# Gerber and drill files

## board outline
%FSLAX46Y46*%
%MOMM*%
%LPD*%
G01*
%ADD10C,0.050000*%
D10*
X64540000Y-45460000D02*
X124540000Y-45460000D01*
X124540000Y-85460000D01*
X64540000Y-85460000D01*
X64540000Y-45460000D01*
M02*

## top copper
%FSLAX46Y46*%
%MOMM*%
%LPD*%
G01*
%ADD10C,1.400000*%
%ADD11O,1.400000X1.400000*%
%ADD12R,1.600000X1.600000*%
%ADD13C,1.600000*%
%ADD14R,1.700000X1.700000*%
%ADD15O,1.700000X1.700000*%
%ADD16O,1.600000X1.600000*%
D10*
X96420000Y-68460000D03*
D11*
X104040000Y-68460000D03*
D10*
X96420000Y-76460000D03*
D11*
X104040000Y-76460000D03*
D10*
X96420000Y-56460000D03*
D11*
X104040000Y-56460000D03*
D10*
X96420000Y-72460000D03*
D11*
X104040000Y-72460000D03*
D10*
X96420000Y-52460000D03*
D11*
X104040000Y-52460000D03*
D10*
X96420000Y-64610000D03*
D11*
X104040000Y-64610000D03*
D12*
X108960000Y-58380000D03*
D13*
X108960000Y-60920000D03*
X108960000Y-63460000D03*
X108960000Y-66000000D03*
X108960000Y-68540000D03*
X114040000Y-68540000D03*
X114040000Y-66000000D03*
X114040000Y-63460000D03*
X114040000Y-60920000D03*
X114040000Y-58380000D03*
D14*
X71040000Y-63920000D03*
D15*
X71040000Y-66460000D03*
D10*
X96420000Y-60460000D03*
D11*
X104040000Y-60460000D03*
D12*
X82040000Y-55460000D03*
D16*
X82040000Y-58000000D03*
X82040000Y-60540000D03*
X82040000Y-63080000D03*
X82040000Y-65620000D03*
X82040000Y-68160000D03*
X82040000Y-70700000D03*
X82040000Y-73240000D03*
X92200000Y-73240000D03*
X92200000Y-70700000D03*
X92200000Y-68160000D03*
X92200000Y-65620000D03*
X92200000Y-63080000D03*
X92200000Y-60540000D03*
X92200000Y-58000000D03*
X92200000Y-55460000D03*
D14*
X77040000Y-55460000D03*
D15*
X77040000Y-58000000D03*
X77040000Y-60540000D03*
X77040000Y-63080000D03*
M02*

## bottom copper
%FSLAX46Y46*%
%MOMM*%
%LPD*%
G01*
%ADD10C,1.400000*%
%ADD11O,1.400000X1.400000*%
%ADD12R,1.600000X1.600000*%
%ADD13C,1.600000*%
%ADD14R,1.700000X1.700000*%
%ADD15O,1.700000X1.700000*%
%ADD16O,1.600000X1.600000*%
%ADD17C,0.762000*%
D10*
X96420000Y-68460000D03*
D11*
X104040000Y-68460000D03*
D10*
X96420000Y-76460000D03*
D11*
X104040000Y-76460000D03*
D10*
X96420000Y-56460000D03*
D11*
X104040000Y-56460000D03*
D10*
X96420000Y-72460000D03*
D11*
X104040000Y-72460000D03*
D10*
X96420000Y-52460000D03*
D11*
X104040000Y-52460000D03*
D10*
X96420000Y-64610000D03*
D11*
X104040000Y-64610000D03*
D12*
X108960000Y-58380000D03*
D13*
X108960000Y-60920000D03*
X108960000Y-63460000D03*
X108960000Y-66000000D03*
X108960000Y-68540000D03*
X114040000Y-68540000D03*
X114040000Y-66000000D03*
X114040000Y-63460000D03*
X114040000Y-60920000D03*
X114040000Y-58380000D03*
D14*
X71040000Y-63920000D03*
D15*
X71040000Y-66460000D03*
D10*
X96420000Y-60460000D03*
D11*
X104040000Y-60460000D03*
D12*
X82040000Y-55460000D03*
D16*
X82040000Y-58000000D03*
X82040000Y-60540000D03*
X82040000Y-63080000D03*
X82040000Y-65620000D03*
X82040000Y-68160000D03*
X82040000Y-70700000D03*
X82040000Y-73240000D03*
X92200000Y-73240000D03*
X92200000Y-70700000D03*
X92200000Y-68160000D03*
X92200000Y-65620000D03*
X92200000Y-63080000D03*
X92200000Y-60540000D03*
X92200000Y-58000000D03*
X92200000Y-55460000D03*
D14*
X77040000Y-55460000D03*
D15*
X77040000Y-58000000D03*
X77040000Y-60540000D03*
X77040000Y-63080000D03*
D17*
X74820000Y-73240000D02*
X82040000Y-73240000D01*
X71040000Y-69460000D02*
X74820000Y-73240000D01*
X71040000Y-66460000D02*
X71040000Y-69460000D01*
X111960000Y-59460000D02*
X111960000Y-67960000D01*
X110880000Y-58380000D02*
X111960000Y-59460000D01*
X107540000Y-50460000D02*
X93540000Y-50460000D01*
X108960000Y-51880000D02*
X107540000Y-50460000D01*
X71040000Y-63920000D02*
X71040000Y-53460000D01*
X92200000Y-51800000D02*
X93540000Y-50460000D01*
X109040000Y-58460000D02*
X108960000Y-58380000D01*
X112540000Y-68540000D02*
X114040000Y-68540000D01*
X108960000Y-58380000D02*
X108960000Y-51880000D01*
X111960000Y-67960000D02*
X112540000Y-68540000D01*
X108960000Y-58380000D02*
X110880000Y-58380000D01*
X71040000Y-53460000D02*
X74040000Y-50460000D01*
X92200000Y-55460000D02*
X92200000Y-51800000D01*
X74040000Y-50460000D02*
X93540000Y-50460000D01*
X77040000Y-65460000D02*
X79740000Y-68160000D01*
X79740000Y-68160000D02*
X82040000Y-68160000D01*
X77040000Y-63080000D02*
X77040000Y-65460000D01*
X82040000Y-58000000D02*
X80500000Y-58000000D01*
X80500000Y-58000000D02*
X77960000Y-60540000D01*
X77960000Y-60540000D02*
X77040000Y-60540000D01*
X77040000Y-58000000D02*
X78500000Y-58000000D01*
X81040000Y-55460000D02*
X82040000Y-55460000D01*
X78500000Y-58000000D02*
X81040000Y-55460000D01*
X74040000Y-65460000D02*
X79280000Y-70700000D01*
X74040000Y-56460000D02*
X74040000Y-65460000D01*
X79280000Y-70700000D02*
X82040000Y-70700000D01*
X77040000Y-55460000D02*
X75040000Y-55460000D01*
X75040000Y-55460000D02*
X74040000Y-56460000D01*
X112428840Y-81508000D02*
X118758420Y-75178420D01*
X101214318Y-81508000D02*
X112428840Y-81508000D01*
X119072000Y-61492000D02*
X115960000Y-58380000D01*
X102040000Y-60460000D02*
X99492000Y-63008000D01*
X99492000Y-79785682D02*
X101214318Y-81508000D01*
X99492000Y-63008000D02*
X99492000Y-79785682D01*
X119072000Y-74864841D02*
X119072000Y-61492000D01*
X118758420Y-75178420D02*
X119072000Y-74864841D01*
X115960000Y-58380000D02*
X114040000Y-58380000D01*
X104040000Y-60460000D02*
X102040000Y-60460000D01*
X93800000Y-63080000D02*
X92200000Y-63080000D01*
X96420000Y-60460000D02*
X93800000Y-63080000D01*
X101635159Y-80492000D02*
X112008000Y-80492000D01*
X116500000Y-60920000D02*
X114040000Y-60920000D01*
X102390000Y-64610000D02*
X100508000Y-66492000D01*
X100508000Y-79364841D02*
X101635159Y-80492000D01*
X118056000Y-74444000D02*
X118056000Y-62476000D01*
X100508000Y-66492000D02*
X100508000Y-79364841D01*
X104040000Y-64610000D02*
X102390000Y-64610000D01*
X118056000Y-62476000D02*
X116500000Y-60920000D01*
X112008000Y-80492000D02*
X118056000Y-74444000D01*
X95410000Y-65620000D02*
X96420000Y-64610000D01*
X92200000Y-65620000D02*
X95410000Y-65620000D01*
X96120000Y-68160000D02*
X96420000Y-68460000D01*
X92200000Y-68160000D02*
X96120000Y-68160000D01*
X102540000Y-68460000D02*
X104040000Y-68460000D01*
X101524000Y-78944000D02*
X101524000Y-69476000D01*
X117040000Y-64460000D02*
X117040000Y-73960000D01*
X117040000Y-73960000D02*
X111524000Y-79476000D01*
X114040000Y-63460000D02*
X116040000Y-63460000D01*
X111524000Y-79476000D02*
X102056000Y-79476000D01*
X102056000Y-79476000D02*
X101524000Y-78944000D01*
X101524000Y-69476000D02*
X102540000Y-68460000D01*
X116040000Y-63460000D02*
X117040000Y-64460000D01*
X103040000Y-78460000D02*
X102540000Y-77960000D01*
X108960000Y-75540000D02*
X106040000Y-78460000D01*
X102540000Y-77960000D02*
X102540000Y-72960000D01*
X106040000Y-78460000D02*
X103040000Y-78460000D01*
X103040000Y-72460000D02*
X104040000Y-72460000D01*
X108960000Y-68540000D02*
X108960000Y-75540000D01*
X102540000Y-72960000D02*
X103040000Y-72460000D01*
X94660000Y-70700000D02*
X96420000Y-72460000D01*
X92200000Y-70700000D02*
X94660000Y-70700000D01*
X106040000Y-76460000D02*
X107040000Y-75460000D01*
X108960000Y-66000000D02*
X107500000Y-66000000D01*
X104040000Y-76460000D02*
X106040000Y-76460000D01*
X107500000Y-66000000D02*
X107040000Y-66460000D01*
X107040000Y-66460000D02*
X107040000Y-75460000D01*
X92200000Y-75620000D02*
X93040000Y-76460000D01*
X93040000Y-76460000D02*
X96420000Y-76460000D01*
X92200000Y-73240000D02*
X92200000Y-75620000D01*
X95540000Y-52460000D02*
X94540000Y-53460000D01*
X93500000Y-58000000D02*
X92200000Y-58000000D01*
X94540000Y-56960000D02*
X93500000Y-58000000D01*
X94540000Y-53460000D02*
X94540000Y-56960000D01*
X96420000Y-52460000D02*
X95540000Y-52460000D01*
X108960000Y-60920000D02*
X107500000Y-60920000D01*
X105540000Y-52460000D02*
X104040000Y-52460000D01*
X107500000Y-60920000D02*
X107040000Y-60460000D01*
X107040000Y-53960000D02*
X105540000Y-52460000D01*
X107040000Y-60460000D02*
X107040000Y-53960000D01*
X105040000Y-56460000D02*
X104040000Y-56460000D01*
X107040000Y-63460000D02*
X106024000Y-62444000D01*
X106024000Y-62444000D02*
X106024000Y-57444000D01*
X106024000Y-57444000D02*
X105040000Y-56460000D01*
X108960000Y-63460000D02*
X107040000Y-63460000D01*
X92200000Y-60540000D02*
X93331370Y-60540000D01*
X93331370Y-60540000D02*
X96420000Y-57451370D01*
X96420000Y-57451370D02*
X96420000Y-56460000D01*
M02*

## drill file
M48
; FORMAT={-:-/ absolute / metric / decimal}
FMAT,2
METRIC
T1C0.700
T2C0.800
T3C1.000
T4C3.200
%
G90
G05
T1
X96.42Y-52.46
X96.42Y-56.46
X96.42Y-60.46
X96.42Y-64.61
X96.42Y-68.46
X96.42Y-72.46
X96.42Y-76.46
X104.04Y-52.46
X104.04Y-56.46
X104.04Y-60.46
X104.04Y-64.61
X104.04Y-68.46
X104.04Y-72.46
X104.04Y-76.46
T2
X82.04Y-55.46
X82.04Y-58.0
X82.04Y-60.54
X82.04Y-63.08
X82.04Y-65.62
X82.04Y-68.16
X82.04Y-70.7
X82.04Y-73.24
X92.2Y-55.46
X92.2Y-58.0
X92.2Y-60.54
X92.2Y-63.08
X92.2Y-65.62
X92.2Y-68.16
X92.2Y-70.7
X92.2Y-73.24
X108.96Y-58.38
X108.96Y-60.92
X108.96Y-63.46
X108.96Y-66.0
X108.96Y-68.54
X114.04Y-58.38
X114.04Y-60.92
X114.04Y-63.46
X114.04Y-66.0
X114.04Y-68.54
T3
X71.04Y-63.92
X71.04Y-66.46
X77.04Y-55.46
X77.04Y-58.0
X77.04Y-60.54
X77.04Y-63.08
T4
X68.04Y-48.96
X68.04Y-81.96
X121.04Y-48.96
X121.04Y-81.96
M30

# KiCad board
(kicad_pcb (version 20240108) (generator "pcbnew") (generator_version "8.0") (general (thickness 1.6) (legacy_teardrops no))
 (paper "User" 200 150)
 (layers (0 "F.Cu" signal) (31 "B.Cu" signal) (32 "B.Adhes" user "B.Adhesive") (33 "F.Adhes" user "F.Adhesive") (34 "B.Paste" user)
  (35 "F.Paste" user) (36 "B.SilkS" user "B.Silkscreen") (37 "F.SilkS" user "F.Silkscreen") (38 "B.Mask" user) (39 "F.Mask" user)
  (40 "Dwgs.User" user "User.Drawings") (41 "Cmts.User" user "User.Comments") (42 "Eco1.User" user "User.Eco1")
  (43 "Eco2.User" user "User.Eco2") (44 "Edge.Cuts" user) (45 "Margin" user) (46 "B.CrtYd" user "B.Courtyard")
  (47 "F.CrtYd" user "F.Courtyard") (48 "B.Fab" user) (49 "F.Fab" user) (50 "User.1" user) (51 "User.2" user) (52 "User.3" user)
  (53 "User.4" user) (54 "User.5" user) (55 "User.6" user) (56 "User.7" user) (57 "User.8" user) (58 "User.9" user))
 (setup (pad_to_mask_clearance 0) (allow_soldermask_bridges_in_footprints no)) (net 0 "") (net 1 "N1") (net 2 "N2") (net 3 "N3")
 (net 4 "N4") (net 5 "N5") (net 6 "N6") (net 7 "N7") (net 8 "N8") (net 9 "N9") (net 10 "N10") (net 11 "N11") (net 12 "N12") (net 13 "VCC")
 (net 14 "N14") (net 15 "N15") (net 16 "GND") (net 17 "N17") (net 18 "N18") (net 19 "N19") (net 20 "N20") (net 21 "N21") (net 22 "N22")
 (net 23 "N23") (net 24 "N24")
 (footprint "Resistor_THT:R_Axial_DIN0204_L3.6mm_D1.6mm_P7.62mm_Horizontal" (layer "F.Cu") (at 96.42 68.46)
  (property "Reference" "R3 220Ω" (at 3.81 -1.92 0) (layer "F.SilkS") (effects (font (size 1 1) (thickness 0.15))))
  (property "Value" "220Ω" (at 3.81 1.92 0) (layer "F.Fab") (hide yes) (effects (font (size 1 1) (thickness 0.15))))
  (pad "1" thru_hole circle (at 0 0) (size 1.4 1.4) (drill 0.7) (layers "*.Cu" "*.Mask") (remove_unused_layers no) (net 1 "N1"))
  (pad "2" thru_hole oval (at 7.62 0) (size 1.4 1.4) (drill 0.7) (layers "*.Cu" "*.Mask") (remove_unused_layers no) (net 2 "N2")))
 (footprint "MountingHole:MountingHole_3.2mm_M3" (layer "F.Cu") (at 68.04 81.96)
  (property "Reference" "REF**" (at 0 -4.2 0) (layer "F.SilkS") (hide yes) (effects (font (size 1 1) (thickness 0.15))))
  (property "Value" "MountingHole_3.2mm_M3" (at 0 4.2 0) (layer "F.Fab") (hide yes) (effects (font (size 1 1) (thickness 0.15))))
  (pad "" np_thru_hole circle (at 0 0) (size 3.2 3.2) (drill 3.2) (layers "*.Cu" "*.Mask")))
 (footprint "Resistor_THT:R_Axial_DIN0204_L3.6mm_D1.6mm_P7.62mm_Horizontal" (layer "F.Cu") (at 96.42 76.46)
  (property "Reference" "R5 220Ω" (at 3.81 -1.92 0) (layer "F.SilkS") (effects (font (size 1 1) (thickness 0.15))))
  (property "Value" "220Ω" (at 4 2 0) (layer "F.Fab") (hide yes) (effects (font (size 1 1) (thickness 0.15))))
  (pad "1" thru_hole circle (at 0 0) (size 1.4 1.4) (drill 0.7) (layers "*.Cu" "*.Mask") (remove_unused_layers no) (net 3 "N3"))
  (pad "2" thru_hole oval (at 7.62 0) (size 1.4 1.4) (drill 0.7) (layers "*.Cu" "*.Mask") (remove_unused_layers no) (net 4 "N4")))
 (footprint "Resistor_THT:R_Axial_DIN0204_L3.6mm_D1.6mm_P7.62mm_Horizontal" (layer "F.Cu") (at 96.42 56.46)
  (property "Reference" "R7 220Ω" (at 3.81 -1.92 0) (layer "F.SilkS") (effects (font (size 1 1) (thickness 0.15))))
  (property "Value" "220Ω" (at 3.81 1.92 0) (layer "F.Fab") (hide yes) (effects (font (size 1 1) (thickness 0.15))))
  (pad "1" thru_hole circle (at 0 0) (size 1.4 1.4) (drill 0.7) (layers "*.Cu" "*.Mask") (remove_unused_layers no) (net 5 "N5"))
  (pad "2" thru_hole oval (at 7.62 0) (size 1.4 1.4) (drill 0.7) (layers "*.Cu" "*.Mask") (remove_unused_layers no) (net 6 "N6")))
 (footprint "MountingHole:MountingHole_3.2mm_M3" (layer "F.Cu") (at 121.04 81.96)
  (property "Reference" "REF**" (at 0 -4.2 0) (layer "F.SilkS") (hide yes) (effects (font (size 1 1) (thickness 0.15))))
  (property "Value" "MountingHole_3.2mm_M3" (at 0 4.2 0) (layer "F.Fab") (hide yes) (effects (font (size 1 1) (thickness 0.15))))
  (pad "" np_thru_hole circle (at 0 0) (size 3.2 3.2) (drill 3.2) (layers "*.Cu" "*.Mask")))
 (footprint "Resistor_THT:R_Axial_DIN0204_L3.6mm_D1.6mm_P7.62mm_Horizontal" (layer "F.Cu") (at 96.42 72.46)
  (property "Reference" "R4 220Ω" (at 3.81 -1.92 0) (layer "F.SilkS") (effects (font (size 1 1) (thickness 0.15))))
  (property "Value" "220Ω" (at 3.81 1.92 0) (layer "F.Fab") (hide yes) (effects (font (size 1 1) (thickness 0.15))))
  (pad "1" thru_hole circle (at 0 0) (size 1.4 1.4) (drill 0.7) (layers "*.Cu" "*.Mask") (remove_unused_layers no) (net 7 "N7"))
  (pad "2" thru_hole oval (at 7.62 0) (size 1.4 1.4) (drill 0.7) (layers "*.Cu" "*.Mask") (remove_unused_layers no) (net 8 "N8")))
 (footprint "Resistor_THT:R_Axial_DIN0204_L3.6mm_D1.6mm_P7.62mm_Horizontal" (layer "F.Cu") (at 96.42 52.46)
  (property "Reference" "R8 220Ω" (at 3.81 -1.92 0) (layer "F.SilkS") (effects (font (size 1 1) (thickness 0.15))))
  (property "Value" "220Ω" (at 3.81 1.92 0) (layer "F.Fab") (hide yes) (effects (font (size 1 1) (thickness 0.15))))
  (pad "1" thru_hole circle (at 0 0) (size 1.4 1.4) (drill 0.7) (layers "*.Cu" "*.Mask") (remove_unused_layers no) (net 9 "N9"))
  (pad "2" thru_hole oval (at 7.62 0) (size 1.4 1.4) (drill 0.7) (layers "*.Cu" "*.Mask") (remove_unused_layers no) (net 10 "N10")))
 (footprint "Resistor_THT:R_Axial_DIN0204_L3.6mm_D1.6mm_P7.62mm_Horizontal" (layer "F.Cu") (at 96.42 64.61)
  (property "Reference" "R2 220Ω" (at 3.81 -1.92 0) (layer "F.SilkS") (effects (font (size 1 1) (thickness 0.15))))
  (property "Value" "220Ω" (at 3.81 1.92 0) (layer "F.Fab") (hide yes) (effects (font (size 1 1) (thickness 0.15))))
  (pad "1" thru_hole circle (at 0 0) (size 1.4 1.4) (drill 0.7) (layers "*.Cu" "*.Mask") (remove_unused_layers no) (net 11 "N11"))
  (pad "2" thru_hole oval (at 7.62 0) (size 1.4 1.4) (drill 0.7) (layers "*.Cu" "*.Mask") (remove_unused_layers no) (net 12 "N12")))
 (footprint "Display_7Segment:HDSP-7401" (layer "F.Cu") (at 108.96 58.38)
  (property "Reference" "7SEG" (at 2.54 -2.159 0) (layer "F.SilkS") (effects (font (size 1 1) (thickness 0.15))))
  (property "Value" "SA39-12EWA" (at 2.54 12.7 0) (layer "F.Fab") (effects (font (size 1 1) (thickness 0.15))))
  (pad "1" thru_hole rect (at 0 0) (size 1.6 1.6) (drill 0.8) (layers "*.Cu" "*.Mask") (remove_unused_layers no) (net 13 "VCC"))
  (pad "2" thru_hole circle (at 0 2.54) (size 1.6 1.6) (drill 0.8) (layers "*.Cu" "*.Mask") (remove_unused_layers no) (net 10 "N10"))
  (pad "3" thru_hole circle (at 0 5.08) (size 1.6 1.6) (drill 0.8) (layers "*.Cu" "*.Mask") (remove_unused_layers no) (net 6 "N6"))
  (pad "4" thru_hole circle (at 0 7.62) (size 1.6 1.6) (drill 0.8) (layers "*.Cu" "*.Mask") (remove_unused_layers no) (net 4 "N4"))
  (pad "5" thru_hole circle (at 0 10.16) (size 1.6 1.6) (drill 0.8) (layers "*.Cu" "*.Mask") (remove_unused_layers no) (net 8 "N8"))
  (pad "6" thru_hole circle (at 5.08 10.16) (size 1.6 1.6) (drill 0.8) (layers "*.Cu" "*.Mask") (remove_unused_layers no) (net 13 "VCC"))
  (pad "7" thru_hole circle (at 5.08 7.62) (size 1.6 1.6) (drill 0.8) (layers "*.Cu" "*.Mask") (remove_unused_layers no) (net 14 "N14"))
  (pad "8" thru_hole circle (at 5.08 5.08) (size 1.6 1.6) (drill 0.8) (layers "*.Cu" "*.Mask") (remove_unused_layers no) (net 2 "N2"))
  (pad "9" thru_hole circle (at 5.08 2.54) (size 1.6 1.6) (drill 0.8) (layers "*.Cu" "*.Mask") (remove_unused_layers no) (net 12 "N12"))
  (pad "10" thru_hole circle (at 5.08 0) (size 1.6 1.6) (drill 0.8) (layers "*.Cu" "*.Mask") (remove_unused_layers no) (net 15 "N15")))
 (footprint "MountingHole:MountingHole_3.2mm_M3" (layer "F.Cu") (at 68.04 48.96)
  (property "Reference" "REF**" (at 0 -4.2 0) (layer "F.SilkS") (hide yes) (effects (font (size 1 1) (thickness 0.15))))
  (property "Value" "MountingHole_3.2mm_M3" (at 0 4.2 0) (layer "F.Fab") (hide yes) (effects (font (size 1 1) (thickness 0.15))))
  (pad "" np_thru_hole circle (at 0 0) (size 3.2 3.2) (drill 3.2) (layers "*.Cu" "*.Mask")))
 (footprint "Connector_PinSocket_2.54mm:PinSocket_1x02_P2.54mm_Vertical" (layer "F.Cu") (at 71.04 63.92)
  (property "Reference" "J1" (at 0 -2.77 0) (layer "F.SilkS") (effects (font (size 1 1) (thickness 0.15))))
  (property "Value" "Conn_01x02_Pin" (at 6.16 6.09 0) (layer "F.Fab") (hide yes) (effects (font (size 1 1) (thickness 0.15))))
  (pad "1" thru_hole rect (at 0 0) (size 1.7 1.7) (drill 1) (layers "*.Cu" "*.Mask") (remove_unused_layers no) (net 13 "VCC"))
  (pad "2" thru_hole oval (at 0 2.54) (size 1.7 1.7) (drill 1) (layers "*.Cu" "*.Mask") (remove_unused_layers no) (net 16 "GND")))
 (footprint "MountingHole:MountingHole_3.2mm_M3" (layer "F.Cu") (at 121.04 48.96)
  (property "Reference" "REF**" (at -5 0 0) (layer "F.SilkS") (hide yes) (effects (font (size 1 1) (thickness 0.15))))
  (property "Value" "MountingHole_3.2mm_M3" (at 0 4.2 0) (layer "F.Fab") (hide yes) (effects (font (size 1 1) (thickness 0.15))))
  (pad "" np_thru_hole circle (at 0 0) (size 3.2 3.2) (drill 3.2) (layers "*.Cu" "*.Mask")))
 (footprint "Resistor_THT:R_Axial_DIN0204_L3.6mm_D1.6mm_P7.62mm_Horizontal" (layer "F.Cu") (at 96.42 60.46)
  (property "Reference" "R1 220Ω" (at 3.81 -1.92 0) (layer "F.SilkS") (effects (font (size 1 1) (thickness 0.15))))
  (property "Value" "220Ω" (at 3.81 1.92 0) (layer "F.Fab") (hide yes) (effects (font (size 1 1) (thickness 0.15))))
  (pad "1" thru_hole circle (at 0 0) (size 1.4 1.4) (drill 0.7) (layers "*.Cu" "*.Mask") (remove_unused_layers no) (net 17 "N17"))
  (pad "2" thru_hole oval (at 7.62 0) (size 1.4 1.4) (drill 0.7) (layers "*.Cu" "*.Mask") (remove_unused_layers no) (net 15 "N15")))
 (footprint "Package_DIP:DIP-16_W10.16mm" (layer "F.Cu") (at 82.04 55.46)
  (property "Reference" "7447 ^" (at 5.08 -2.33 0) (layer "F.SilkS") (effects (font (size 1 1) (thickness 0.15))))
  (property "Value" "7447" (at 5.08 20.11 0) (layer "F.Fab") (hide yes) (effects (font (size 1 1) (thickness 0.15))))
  (pad "1" thru_hole rect (at 0 0) (size 1.6 1.6) (drill 0.8) (layers "*.Cu" "*.Mask") (remove_unused_layers no) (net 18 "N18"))
  (pad "2" thru_hole oval (at 0 2.54) (size 1.6 1.6) (drill 0.8) (layers "*.Cu" "*.Mask") (remove_unused_layers no) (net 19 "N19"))
  (pad "3" thru_hole oval (at 0 5.08) (size 1.6 1.6) (drill 0.8) (layers "*.Cu" "*.Mask") (remove_unused_layers no) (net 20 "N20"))
  (pad "4" thru_hole oval (at 0 7.62) (size 1.6 1.6) (drill 0.8) (layers "*.Cu" "*.Mask") (remove_unused_layers no) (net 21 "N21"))
  (pad "5" thru_hole oval (at 0 10.16) (size 1.6 1.6) (drill 0.8) (layers "*.Cu" "*.Mask") (remove_unused_layers no) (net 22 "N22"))
  (pad "6" thru_hole oval (at 0 12.7) (size 1.6 1.6) (drill 0.8) (layers "*.Cu" "*.Mask") (remove_unused_layers no) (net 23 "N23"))
  (pad "7" thru_hole oval (at 0 15.24) (size 1.6 1.6) (drill 0.8) (layers "*.Cu" "*.Mask") (remove_unused_layers no) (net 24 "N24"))
  (pad "8" thru_hole oval (at 0 17.78) (size 1.6 1.6) (drill 0.8) (layers "*.Cu" "*.Mask") (remove_unused_layers no) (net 16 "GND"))
  (pad "9" thru_hole oval (at 10.16 17.78) (size 1.6 1.6) (drill 0.8) (layers "*.Cu" "*.Mask") (remove_unused_layers no) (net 3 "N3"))
  (pad "10" thru_hole oval (at 10.16 15.24) (size 1.6 1.6) (drill 0.8) (layers "*.Cu" "*.Mask") (remove_unused_layers no) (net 7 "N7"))
  (pad "11" thru_hole oval (at 10.16 12.7) (size 1.6 1.6) (drill 0.8) (layers "*.Cu" "*.Mask") (remove_unused_layers no) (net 1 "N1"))
  (pad "12" thru_hole oval (at 10.16 10.16) (size 1.6 1.6) (drill 0.8) (layers "*.Cu" "*.Mask") (remove_unused_layers no) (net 11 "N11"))
  (pad "13" thru_hole oval (at 10.16 7.62) (size 1.6 1.6) (drill 0.8) (layers "*.Cu" "*.Mask") (remove_unused_layers no) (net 17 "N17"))
  (pad "14" thru_hole oval (at 10.16 5.08) (size 1.6 1.6) (drill 0.8) (layers "*.Cu" "*.Mask") (remove_unused_layers no) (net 5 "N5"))
  (pad "15" thru_hole oval (at 10.16 2.54) (size 1.6 1.6) (drill 0.8) (layers "*.Cu" "*.Mask") (remove_unused_layers no) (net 9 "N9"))
  (pad "16" thru_hole oval (at 10.16 0) (size 1.6 1.6) (drill 0.8) (layers "*.Cu" "*.Mask") (remove_unused_layers no) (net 13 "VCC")))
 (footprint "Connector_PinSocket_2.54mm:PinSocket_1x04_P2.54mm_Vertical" (layer "F.Cu") (at 77.04 55.46)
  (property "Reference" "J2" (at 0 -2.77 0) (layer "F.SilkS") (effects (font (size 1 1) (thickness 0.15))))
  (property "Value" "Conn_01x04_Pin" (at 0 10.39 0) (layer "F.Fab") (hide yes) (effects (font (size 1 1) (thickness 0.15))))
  (pad "1" thru_hole rect (at 0 0) (size 1.7 1.7) (drill 1) (layers "*.Cu" "*.Mask") (remove_unused_layers no) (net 24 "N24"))
  (pad "2" thru_hole oval (at 0 2.54) (size 1.7 1.7) (drill 1) (layers "*.Cu" "*.Mask") (remove_unused_layers no) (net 18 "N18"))
  (pad "3" thru_hole oval (at 0 5.08) (size 1.7 1.7) (drill 1) (layers "*.Cu" "*.Mask") (remove_unused_layers no) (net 19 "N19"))
  (pad "4" thru_hole oval (at 0 7.62) (size 1.7 1.7) (drill 1) (layers "*.Cu" "*.Mask") (remove_unused_layers no) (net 23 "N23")))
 (gr_rect (start 64.54 45.46) (end 124.54 85.46) (stroke (width 0.05) (type default)) (fill none) (layer "Edge.Cuts"))
 (segment (start 74.82 73.24) (end 82.04 73.24) (width 0.762) (layer "B.Cu") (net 16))
 (segment (start 71.04 69.46) (end 74.82 73.24) (width 0.762) (layer "B.Cu") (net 16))
 (segment (start 71.04 66.46) (end 71.04 69.46) (width 0.762) (layer "B.Cu") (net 16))
 (segment (start 111.96 59.46) (end 111.96 67.96) (width 0.762) (layer "B.Cu") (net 13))
 (segment (start 110.88 58.38) (end 111.96 59.46) (width 0.762) (layer "B.Cu") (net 13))
 (segment (start 107.54 50.46) (end 93.54 50.46) (width 0.762) (layer "B.Cu") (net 13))
 (segment (start 108.96 51.88) (end 107.54 50.46) (width 0.762) (layer "B.Cu") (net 13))
 (segment (start 71.04 63.92) (end 71.04 53.46) (width 0.762) (layer "B.Cu") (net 13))
 (segment (start 92.2 51.8) (end 93.54 50.46) (width 0.762) (layer "B.Cu") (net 13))
 (segment (start 109.04 58.46) (end 108.96 58.38) (width 0.762) (layer "B.Cu") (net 13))
 (segment (start 112.54 68.54) (end 114.04 68.54) (width 0.762) (layer "B.Cu") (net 13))
 (segment (start 108.96 58.38) (end 108.96 51.88) (width 0.762) (layer "B.Cu") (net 13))
 (segment (start 111.96 67.96) (end 112.54 68.54) (width 0.762) (layer "B.Cu") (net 13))
 (segment (start 108.96 58.38) (end 110.88 58.38) (width 0.762) (layer "B.Cu") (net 13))
 (segment (start 71.04 53.46) (end 74.04 50.46) (width 0.762) (layer "B.Cu") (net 13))
 (segment (start 92.2 55.46) (end 92.2 51.8) (width 0.762) (layer "B.Cu") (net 13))
 (segment (start 74.04 50.46) (end 93.54 50.46) (width 0.762) (layer "B.Cu") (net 13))
 (segment (start 77.04 65.46) (end 79.74 68.16) (width 0.762) (layer "B.Cu") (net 23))
 (segment (start 79.74 68.16) (end 82.04 68.16) (width 0.762) (layer "B.Cu") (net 23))
 (segment (start 77.04 63.08) (end 77.04 65.46) (width 0.762) (layer "B.Cu") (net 23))
 (segment (start 82.04 58) (end 80.5 58) (width 0.762) (layer "B.Cu") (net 19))
 (segment (start 80.5 58) (end 77.96 60.54) (width 0.762) (layer "B.Cu") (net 19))
 (segment (start 77.96 60.54) (end 77.04 60.54) (width 0.762) (layer "B.Cu") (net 19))
 (segment (start 77.04 58) (end 78.5 58) (width 0.762) (layer "B.Cu") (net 18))
 (segment (start 81.04 55.46) (end 82.04 55.46) (width 0.762) (layer "B.Cu") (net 18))
 (segment (start 78.5 58) (end 81.04 55.46) (width 0.762) (layer "B.Cu") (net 18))
 (segment (start 74.04 65.46) (end 79.28 70.7) (width 0.762) (layer "B.Cu") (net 24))
 (segment (start 74.04 56.46) (end 74.04 65.46) (width 0.762) (layer "B.Cu") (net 24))
 (segment (start 79.28 70.7) (end 82.04 70.7) (width 0.762) (layer "B.Cu") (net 24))
 (segment (start 77.04 55.46) (end 75.04 55.46) (width 0.762) (layer "B.Cu") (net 24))
 (segment (start 75.04 55.46) (end 74.04 56.46) (width 0.762) (layer "B.Cu") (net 24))
 (segment (start 112.42884 81.508) (end 118.75842 75.17842) (width 0.762) (layer "B.Cu") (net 15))
 (segment (start 101.214318 81.508) (end 112.42884 81.508) (width 0.762) (layer "B.Cu") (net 15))
 (segment (start 119.072 61.492) (end 115.96 58.38) (width 0.762) (layer "B.Cu") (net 15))
 (segment (start 102.04 60.46) (end 99.492 63.008) (width 0.762) (layer "B.Cu") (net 15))
 (segment (start 99.492 79.785682) (end 101.214318 81.508) (width 0.762) (layer "B.Cu") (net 15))
 (segment (start 99.492 63.008) (end 99.492 79.785682) (width 0.762) (layer "B.Cu") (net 15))
 (segment (start 119.072 74.864841) (end 119.072 61.492) (width 0.762) (layer "B.Cu") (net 15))
 (segment (start 118.75842 75.17842) (end 119.072 74.864841) (width 0.762) (layer "B.Cu") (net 15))
 (segment (start 115.96 58.38) (end 114.04 58.38) (width 0.762) (layer "B.Cu") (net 15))
 (segment (start 104.04 60.46) (end 102.04 60.46) (width 0.762) (layer "B.Cu") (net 15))
 (segment (start 93.8 63.08) (end 92.2 63.08) (width 0.762) (layer "B.Cu") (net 17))
 (segment (start 96.42 60.46) (end 93.8 63.08) (width 0.762) (layer "B.Cu") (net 17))
 (segment (start 101.635159 80.492) (end 112.008 80.492) (width 0.762) (layer "B.Cu") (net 12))
 (segment (start 116.5 60.92) (end 114.04 60.92) (width 0.762) (layer "B.Cu") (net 12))
 (segment (start 102.39 64.61) (end 100.508 66.492) (width 0.762) (layer "B.Cu") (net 12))
 (segment (start 100.508 79.364841) (end 101.635159 80.492) (width 0.762) (layer "B.Cu") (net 12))
 (segment (start 118.056 74.444) (end 118.056 62.476) (width 0.762) (layer "B.Cu") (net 12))
 (segment (start 100.508 66.492) (end 100.508 79.364841) (width 0.762) (layer "B.Cu") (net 12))
 (segment (start 104.04 64.61) (end 102.39 64.61) (width 0.762) (layer "B.Cu") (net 12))
 (segment (start 118.056 62.476) (end 116.5 60.92) (width 0.762) (layer "B.Cu") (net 12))
 (segment (start 112.008 80.492) (end 118.056 74.444) (width 0.762) (layer "B.Cu") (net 12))
 (segment (start 95.41 65.62) (end 96.42 64.61) (width 0.762) (layer "B.Cu") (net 11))
 (segment (start 92.2 65.62) (end 95.41 65.62) (width 0.762) (layer "B.Cu") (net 11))
 (segment (start 96.12 68.16) (end 96.42 68.46) (width 0.762) (layer "B.Cu") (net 1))
 (segment (start 92.2 68.16) (end 96.12 68.16) (width 0.762) (layer "B.Cu") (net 1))
 (segment (start 102.54 68.46) (end 104.04 68.46) (width 0.762) (layer "B.Cu") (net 2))
 (segment (start 101.524 78.944) (end 101.524 69.476) (width 0.762) (layer "B.Cu") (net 2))
 (segment (start 117.04 64.46) (end 117.04 73.96) (width 0.762) (layer "B.Cu") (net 2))
 (segment (start 117.04 73.96) (end 111.524 79.476) (width 0.762) (layer "B.Cu") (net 2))
 (segment (start 114.04 63.46) (end 116.04 63.46) (width 0.762) (layer "B.Cu") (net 2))
 (segment (start 111.524 79.476) (end 102.056 79.476) (width 0.762) (layer "B.Cu") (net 2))
 (segment (start 102.056 79.476) (end 101.524 78.944) (width 0.762) (layer "B.Cu") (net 2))
 (segment (start 101.524 69.476) (end 102.54 68.46) (width 0.762) (layer "B.Cu") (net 2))
 (segment (start 116.04 63.46) (end 117.04 64.46) (width 0.762) (layer "B.Cu") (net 2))
 (segment (start 103.04 78.46) (end 102.54 77.96) (width 0.762) (layer "B.Cu") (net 8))
 (segment (start 108.96 75.54) (end 106.04 78.46) (width 0.762) (layer "B.Cu") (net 8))
 (segment (start 102.54 77.96) (end 102.54 72.96) (width 0.762) (layer "B.Cu") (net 8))
 (segment (start 106.04 78.46) (end 103.04 78.46) (width 0.762) (layer "B.Cu") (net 8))
 (segment (start 103.04 72.46) (end 104.04 72.46) (width 0.762) (layer "B.Cu") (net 8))
 (segment (start 108.96 68.54) (end 108.96 75.54) (width 0.762) (layer "B.Cu") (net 8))
 (segment (start 102.54 72.96) (end 103.04 72.46) (width 0.762) (layer "B.Cu") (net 8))
 (segment (start 94.66 70.7) (end 96.42 72.46) (width 0.762) (layer "B.Cu") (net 7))
 (segment (start 92.2 70.7) (end 94.66 70.7) (width 0.762) (layer "B.Cu") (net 7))
 (segment (start 106.04 76.46) (end 107.04 75.46) (width 0.762) (layer "B.Cu") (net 4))
 (segment (start 108.96 66) (end 107.5 66) (width 0.762) (layer "B.Cu") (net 4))
 (segment (start 104.04 76.46) (end 106.04 76.46) (width 0.762) (layer "B.Cu") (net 4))
 (segment (start 107.5 66) (end 107.04 66.46) (width 0.762) (layer "B.Cu") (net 4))
 (segment (start 107.04 66.46) (end 107.04 75.46) (width 0.762) (layer "B.Cu") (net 4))
 (segment (start 92.2 75.62) (end 93.04 76.46) (width 0.762) (layer "B.Cu") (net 3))
 (segment (start 93.04 76.46) (end 96.42 76.46) (width 0.762) (layer "B.Cu") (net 3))
 (segment (start 92.2 73.24) (end 92.2 75.62) (width 0.762) (layer "B.Cu") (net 3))
 (segment (start 95.54 52.46) (end 94.54 53.46) (width 0.762) (layer "B.Cu") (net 9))
 (segment (start 93.5 58) (end 92.2 58) (width 0.762) (layer "B.Cu") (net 9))
 (segment (start 94.54 56.96) (end 93.5 58) (width 0.762) (layer "B.Cu") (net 9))
 (segment (start 94.54 53.46) (end 94.54 56.96) (width 0.762) (layer "B.Cu") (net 9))
 (segment (start 96.42 52.46) (end 95.54 52.46) (width 0.762) (layer "B.Cu") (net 9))
 (segment (start 108.96 60.92) (end 107.5 60.92) (width 0.762) (layer "B.Cu") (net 10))
 (segment (start 105.54 52.46) (end 104.04 52.46) (width 0.762) (layer "B.Cu") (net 10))
 (segment (start 107.5 60.92) (end 107.04 60.46) (width 0.762) (layer "B.Cu") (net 10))
 (segment (start 107.04 53.96) (end 105.54 52.46) (width 0.762) (layer "B.Cu") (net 10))
 (segment (start 107.04 60.46) (end 107.04 53.96) (width 0.762) (layer "B.Cu") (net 10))
 (segment (start 105.04 56.46) (end 104.04 56.46) (width 0.762) (layer "B.Cu") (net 6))
 (segment (start 107.04 63.46) (end 106.024 62.444) (width 0.762) (layer "B.Cu") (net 6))
 (segment (start 106.024 62.444) (end 106.024 57.444) (width 0.762) (layer "B.Cu") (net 6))
 (segment (start 106.024 57.444) (end 105.04 56.46) (width 0.762) (layer "B.Cu") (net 6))
 (segment (start 108.96 63.46) (end 107.04 63.46) (width 0.762) (layer "B.Cu") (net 6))
 (segment (start 92.2 60.54) (end 93.33137 60.54) (width 0.762) (layer "B.Cu") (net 5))
 (segment (start 93.33137 60.54) (end 96.42 57.45137) (width 0.762) (layer "B.Cu") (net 5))
 (segment (start 96.42 57.45137) (end 96.42 56.46) (width 0.762) (layer "B.Cu") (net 5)))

